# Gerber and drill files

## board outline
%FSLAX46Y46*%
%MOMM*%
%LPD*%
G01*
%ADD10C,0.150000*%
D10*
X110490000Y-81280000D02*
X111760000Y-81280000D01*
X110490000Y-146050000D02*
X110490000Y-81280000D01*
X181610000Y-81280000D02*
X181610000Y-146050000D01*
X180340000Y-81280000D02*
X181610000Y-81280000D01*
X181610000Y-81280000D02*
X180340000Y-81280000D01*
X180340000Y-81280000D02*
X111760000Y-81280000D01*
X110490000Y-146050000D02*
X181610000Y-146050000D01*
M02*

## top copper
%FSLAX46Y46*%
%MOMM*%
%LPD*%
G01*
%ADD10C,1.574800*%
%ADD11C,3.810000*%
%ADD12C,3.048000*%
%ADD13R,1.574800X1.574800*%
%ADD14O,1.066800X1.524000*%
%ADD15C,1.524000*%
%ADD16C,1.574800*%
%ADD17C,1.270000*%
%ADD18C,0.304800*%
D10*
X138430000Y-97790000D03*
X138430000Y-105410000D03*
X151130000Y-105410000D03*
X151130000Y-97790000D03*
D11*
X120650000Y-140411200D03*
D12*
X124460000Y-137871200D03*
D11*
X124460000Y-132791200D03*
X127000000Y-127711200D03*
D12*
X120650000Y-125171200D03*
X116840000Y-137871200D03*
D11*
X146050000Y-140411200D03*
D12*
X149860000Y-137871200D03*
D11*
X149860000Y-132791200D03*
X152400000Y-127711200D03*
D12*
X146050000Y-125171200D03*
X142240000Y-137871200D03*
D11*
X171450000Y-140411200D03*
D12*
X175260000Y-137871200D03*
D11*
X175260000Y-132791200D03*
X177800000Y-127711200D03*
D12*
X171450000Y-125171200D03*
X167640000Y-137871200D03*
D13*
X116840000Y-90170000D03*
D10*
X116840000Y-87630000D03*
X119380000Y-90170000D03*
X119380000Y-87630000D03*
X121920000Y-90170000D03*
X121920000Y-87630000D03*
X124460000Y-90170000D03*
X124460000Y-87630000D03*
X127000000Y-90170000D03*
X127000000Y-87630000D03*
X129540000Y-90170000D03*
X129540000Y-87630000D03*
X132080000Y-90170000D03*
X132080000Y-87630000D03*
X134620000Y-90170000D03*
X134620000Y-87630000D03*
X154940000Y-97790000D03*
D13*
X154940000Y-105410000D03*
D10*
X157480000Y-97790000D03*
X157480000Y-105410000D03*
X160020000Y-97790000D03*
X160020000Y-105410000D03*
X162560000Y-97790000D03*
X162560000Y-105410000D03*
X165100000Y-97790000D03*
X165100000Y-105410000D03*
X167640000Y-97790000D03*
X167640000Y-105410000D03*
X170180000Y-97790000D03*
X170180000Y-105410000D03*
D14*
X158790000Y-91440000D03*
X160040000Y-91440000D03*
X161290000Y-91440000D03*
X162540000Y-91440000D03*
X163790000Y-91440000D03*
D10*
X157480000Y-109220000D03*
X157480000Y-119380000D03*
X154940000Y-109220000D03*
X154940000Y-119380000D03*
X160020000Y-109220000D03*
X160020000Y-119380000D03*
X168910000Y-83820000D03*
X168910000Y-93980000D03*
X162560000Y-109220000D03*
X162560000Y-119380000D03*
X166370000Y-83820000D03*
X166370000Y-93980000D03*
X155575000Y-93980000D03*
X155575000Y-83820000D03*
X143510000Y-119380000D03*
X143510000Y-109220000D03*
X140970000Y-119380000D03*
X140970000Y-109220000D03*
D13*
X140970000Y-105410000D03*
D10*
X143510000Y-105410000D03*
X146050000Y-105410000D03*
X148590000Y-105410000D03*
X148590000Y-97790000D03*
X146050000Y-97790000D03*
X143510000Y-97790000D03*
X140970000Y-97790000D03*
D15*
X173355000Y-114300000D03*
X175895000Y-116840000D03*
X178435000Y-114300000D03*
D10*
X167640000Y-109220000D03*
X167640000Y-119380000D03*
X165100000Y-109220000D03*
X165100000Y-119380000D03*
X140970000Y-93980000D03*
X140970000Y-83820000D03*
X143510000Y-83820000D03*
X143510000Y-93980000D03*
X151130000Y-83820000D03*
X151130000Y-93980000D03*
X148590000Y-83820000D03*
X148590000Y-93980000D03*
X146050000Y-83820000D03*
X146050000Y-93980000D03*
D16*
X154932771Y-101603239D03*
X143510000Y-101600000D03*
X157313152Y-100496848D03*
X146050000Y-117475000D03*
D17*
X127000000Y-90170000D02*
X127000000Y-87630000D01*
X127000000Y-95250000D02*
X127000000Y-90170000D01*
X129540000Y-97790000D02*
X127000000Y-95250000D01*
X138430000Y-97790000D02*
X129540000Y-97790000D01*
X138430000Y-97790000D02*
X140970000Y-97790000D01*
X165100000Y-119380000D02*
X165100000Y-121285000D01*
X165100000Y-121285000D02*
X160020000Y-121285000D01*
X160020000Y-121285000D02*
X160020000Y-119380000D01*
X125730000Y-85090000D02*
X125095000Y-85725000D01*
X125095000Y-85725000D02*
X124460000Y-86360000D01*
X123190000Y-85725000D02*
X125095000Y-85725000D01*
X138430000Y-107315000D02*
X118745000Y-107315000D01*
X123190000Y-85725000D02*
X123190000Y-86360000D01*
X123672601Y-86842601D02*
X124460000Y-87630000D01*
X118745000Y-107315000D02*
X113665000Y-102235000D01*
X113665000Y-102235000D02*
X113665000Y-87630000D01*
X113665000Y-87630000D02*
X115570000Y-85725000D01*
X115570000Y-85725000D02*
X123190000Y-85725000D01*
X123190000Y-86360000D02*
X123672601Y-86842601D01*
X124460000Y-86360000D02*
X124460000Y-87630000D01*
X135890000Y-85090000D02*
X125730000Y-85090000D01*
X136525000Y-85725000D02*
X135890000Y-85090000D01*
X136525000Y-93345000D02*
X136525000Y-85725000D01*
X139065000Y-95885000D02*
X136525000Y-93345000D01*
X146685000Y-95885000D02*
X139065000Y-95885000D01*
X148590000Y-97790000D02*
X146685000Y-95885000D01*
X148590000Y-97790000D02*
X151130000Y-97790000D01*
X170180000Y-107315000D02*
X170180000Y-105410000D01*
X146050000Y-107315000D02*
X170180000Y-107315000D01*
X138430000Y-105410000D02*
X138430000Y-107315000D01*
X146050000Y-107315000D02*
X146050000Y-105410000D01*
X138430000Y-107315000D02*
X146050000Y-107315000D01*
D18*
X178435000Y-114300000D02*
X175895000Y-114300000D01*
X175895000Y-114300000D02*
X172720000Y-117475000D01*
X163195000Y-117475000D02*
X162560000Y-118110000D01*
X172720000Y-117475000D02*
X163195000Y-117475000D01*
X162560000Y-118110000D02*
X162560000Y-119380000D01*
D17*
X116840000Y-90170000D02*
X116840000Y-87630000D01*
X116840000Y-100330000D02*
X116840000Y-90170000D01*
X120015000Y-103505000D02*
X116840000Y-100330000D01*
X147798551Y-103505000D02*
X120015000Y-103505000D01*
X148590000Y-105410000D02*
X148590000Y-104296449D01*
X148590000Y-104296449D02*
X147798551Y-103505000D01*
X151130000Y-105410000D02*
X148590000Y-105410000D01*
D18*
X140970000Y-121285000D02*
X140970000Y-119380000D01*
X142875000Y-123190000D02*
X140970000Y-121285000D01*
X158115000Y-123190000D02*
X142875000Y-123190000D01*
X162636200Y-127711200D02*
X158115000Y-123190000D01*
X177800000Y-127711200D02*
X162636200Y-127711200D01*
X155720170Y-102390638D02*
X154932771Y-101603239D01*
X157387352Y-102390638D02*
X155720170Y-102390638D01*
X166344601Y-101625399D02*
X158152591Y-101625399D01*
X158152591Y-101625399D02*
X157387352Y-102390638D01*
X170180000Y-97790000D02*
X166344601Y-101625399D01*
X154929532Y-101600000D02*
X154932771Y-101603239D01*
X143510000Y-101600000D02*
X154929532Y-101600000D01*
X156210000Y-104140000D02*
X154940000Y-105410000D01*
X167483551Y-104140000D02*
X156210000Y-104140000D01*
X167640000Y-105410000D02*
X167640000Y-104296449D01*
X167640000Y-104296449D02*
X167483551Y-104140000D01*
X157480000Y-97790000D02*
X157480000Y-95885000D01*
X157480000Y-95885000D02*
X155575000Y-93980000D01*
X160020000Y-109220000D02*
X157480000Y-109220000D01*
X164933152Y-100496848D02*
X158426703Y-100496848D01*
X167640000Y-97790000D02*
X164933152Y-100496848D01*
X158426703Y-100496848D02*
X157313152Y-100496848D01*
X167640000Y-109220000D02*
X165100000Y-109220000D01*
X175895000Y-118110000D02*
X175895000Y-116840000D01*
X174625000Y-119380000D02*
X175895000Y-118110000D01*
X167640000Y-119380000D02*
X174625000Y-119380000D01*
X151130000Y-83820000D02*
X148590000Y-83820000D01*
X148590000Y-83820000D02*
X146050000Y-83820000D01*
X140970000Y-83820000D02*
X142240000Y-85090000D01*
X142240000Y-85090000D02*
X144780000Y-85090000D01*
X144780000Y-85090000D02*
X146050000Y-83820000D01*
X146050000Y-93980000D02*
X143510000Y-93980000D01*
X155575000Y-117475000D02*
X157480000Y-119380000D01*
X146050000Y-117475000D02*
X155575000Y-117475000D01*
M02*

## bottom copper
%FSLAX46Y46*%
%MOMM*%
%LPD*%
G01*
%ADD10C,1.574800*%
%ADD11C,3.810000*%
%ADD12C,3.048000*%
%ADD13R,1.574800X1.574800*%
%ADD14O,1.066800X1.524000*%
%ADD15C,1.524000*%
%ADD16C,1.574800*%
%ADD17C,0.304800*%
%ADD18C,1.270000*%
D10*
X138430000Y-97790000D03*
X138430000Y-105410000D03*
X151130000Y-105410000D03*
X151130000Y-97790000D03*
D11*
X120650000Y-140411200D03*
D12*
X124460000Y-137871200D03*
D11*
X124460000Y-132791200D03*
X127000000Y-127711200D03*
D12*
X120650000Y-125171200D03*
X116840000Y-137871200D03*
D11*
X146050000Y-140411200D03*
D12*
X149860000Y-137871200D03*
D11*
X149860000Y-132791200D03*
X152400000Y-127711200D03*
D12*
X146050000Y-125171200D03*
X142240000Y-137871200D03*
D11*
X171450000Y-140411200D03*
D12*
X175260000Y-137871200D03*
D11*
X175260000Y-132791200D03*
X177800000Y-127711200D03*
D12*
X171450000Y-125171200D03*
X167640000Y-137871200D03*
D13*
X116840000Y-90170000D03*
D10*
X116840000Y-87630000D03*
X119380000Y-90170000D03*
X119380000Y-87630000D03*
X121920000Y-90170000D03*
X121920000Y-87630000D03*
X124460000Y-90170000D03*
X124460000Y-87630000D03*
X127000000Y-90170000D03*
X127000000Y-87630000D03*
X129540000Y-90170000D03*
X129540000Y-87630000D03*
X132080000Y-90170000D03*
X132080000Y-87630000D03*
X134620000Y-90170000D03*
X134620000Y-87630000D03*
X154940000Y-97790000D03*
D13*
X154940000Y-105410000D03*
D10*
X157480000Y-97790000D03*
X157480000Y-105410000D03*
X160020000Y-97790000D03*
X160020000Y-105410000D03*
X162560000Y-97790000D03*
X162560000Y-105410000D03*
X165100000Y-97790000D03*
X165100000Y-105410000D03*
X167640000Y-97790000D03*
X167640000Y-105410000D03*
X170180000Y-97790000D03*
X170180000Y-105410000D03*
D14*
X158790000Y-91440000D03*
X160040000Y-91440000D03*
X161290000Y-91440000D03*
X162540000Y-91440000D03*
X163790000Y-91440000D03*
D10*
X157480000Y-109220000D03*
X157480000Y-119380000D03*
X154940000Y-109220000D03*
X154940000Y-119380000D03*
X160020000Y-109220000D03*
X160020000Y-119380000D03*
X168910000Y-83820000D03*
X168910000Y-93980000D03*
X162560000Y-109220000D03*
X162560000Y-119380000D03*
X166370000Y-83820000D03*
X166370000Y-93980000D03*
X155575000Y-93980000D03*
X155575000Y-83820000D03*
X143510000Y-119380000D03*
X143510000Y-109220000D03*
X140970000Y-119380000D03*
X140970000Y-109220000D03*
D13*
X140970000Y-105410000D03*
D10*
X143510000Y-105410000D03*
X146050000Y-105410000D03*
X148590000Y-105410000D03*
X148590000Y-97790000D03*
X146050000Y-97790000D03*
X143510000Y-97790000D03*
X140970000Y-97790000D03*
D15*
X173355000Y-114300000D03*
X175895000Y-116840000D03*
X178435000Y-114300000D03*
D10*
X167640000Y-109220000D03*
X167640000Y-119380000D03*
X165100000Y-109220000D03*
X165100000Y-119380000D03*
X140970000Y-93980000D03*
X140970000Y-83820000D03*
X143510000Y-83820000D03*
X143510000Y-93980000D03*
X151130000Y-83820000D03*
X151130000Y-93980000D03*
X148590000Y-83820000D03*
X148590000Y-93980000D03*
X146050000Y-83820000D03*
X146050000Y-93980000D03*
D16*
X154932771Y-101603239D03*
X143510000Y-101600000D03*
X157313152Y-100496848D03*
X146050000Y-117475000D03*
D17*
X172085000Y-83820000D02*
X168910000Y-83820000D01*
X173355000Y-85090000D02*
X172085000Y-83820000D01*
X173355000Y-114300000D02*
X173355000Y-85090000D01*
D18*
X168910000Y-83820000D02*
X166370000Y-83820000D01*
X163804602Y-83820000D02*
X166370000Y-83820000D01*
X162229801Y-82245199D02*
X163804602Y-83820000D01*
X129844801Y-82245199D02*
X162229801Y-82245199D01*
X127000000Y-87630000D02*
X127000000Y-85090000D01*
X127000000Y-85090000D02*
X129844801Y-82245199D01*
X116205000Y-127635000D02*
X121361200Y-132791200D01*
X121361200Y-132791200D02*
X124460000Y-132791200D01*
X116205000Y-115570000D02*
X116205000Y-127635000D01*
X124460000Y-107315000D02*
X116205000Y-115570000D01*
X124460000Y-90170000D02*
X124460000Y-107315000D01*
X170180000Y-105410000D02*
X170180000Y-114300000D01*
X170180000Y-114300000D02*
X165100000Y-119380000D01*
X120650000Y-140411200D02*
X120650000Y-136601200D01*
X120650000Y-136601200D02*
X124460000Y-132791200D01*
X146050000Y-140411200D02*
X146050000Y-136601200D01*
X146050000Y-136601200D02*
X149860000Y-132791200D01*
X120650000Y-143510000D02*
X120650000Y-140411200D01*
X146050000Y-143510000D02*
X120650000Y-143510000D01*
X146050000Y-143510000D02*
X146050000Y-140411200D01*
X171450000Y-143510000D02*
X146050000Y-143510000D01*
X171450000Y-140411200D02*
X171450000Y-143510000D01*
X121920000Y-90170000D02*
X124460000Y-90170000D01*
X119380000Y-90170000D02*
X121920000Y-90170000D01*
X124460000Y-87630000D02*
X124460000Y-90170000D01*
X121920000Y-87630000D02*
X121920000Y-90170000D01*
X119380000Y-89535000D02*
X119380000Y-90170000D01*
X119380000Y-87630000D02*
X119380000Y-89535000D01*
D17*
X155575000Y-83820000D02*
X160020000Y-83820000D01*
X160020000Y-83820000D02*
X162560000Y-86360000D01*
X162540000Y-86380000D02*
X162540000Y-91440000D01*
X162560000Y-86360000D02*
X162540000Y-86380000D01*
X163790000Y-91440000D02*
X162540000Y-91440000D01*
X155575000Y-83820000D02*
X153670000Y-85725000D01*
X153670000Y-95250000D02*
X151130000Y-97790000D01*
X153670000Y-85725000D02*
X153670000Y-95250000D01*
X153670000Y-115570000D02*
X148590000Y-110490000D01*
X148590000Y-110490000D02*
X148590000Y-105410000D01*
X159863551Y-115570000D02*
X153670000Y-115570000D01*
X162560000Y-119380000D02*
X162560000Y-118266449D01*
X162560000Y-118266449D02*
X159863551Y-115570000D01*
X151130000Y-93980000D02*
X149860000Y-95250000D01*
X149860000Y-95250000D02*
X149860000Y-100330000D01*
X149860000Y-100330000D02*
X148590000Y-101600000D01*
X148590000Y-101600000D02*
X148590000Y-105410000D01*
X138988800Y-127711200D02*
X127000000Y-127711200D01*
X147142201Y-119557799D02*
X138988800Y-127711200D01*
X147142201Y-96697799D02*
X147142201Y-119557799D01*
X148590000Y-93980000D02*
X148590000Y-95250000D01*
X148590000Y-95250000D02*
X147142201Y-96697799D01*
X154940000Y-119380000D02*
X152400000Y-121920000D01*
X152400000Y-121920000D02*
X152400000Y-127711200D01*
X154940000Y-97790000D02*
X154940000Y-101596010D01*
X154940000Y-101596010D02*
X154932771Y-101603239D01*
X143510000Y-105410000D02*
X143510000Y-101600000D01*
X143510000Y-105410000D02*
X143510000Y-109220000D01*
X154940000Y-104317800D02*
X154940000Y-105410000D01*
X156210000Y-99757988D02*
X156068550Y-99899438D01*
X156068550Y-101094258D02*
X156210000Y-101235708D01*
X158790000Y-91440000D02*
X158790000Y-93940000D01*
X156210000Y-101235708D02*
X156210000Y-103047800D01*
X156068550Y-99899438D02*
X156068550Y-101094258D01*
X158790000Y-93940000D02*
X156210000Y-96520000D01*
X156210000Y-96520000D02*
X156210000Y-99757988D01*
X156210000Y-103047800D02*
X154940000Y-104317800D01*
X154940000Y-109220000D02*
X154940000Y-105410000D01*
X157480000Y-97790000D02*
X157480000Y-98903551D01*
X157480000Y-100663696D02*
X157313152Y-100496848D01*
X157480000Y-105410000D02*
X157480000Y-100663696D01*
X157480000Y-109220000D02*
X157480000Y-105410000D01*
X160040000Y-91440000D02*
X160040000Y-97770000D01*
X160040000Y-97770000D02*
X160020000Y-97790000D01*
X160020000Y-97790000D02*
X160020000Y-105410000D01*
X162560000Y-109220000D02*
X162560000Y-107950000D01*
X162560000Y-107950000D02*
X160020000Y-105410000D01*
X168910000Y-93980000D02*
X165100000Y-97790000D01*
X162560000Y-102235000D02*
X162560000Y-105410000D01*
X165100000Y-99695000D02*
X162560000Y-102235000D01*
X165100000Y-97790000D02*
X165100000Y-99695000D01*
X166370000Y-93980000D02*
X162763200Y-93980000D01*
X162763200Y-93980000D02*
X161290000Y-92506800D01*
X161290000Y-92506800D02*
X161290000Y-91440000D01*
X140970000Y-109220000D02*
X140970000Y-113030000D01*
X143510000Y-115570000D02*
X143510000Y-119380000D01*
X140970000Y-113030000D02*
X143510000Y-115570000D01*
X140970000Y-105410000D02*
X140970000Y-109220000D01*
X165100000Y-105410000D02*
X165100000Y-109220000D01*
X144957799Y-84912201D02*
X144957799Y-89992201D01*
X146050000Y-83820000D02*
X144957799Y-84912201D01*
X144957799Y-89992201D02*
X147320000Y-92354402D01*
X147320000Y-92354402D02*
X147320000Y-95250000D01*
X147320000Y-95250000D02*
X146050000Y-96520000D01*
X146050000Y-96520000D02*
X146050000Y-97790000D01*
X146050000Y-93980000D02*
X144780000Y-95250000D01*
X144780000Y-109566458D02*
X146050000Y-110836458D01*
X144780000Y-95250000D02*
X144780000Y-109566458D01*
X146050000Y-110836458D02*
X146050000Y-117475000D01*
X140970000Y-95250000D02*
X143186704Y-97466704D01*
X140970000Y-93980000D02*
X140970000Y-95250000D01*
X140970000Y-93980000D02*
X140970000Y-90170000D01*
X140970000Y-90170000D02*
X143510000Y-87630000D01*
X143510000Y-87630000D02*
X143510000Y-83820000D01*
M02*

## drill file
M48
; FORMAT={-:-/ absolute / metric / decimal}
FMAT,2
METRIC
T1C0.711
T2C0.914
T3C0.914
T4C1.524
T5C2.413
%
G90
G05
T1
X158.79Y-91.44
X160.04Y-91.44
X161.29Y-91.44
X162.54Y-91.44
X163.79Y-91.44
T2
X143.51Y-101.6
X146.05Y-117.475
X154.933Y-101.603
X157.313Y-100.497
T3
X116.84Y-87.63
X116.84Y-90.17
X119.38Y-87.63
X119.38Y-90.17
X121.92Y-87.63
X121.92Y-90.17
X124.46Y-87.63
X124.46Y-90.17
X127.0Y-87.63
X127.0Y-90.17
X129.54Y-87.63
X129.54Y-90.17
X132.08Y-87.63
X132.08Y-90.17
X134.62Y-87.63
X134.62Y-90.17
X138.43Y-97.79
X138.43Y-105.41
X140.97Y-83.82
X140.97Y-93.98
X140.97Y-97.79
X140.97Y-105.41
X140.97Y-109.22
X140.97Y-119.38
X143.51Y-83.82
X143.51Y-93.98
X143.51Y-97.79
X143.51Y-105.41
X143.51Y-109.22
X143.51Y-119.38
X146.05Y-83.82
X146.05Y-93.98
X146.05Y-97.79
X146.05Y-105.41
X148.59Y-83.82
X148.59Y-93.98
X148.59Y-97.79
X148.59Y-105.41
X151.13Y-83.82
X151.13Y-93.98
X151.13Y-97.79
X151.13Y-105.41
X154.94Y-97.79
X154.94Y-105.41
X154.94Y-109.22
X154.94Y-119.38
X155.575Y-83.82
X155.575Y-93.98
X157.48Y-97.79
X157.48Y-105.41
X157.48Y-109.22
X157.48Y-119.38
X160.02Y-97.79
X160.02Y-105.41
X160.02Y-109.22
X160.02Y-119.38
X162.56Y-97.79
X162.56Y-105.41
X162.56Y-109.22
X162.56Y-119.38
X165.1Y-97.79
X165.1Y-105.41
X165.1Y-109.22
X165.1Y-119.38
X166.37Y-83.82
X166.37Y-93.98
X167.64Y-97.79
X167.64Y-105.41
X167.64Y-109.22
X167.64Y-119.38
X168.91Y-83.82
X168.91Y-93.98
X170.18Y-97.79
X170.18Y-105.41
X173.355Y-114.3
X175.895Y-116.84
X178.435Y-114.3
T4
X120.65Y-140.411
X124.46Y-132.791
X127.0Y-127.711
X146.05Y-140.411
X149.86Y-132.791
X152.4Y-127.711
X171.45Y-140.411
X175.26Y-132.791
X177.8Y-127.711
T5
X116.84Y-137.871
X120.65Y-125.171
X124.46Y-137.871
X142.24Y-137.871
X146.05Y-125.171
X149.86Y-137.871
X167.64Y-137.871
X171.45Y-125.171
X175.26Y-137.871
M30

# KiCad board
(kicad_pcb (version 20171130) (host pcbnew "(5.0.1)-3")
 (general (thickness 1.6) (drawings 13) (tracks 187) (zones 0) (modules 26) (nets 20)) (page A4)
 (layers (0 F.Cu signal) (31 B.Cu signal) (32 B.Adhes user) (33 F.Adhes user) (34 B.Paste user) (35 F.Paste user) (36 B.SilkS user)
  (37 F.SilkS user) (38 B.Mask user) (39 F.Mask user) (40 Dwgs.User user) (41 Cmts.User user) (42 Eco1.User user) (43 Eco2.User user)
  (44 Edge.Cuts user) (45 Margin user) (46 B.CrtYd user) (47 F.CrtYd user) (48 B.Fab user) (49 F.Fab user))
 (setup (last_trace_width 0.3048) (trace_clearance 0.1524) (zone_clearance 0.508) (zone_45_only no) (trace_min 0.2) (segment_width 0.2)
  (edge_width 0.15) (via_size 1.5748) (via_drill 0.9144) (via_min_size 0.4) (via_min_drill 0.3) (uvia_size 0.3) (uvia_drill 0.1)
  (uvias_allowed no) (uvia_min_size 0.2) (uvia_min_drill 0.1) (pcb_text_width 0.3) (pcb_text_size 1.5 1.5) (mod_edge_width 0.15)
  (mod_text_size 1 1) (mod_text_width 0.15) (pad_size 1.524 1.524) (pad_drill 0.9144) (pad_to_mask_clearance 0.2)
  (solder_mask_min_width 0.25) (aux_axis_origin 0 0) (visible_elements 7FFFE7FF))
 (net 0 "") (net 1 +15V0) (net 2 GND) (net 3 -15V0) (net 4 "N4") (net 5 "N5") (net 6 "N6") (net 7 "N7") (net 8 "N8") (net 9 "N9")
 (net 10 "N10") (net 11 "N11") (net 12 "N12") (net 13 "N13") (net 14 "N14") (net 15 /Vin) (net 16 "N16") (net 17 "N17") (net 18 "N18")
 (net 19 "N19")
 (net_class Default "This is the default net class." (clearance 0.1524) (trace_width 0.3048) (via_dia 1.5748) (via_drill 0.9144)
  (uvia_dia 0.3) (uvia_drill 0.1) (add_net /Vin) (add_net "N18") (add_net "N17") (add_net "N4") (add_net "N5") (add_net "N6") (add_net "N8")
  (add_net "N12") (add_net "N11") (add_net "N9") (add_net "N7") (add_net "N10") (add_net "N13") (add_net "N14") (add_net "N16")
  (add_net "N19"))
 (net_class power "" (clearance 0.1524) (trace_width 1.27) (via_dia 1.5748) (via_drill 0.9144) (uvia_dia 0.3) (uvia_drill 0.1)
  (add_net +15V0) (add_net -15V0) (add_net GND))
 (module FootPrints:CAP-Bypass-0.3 (layer F.Cu) (at 138.43 101.6 270)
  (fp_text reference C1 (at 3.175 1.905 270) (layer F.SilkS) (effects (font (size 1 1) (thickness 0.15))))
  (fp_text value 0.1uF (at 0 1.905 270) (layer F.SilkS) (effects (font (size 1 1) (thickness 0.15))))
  (pad 1 thru_hole circle (at -3.81 0 270) (size 1.5748 1.5748) (drill 0.9144) (layers *.Cu *.Mask F.SilkS) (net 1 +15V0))
  (pad 2 thru_hole circle (at 3.81 0 270) (size 1.5748 1.5748) (drill 0.9144) (layers *.Cu *.Mask F.SilkS) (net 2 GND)))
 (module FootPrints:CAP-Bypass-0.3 (layer F.Cu) (at 151.13 101.6 90)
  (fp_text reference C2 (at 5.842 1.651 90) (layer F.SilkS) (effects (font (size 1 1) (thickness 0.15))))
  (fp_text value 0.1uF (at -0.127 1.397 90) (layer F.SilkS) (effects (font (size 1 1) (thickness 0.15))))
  (pad 1 thru_hole circle (at -3.81 0 90) (size 1.5748 1.5748) (drill 0.9144) (layers *.Cu *.Mask F.SilkS) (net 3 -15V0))
  (pad 2 thru_hole circle (at 3.81 0 90) (size 1.5748 1.5748) (drill 0.9144) (layers *.Cu *.Mask F.SilkS) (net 2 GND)))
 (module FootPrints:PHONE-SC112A (layer F.Cu) (at 120.65 146.05 270)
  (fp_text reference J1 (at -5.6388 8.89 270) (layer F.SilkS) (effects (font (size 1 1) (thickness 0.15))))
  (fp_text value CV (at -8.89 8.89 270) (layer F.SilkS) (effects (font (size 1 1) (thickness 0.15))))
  (pad 1 thru_hole circle (at -5.6388 0 270) (size 3.81 3.81) (drill 1.524) (layers *.Cu *.Mask F.SilkS) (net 2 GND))
  (pad "" thru_hole circle (at -8.1788 -3.81 270) (size 3.048 3.048) (drill 2.413) (layers *.Cu *.Mask F.SilkS))
  (pad 2 thru_hole circle (at -13.2588 -3.81 270) (size 3.81 3.81) (drill 1.524) (layers *.Cu *.Mask F.SilkS) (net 2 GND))
  (pad 3 thru_hole circle (at -18.3388 -6.35 270) (size 3.81 3.81) (drill 1.524) (layers *.Cu *.Mask F.SilkS) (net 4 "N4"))
  (pad "" thru_hole circle (at -20.8788 0 270) (size 3.048 3.048) (drill 2.413) (layers *.Cu *.Mask F.SilkS))
  (pad "" thru_hole circle (at -8.1788 3.81 270) (size 3.048 3.048) (drill 2.413) (layers *.Cu *.Mask F.SilkS)))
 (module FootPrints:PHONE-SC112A (layer F.Cu) (at 146.05 146.05 270)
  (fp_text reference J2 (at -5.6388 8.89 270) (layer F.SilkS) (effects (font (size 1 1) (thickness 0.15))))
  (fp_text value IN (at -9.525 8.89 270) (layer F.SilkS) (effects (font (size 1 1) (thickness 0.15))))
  (pad 1 thru_hole circle (at -5.6388 0 270) (size 3.81 3.81) (drill 1.524) (layers *.Cu *.Mask F.SilkS) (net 2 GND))
  (pad "" thru_hole circle (at -8.1788 -3.81 270) (size 3.048 3.048) (drill 2.413) (layers *.Cu *.Mask F.SilkS))
  (pad 2 thru_hole circle (at -13.2588 -3.81 270) (size 3.81 3.81) (drill 1.524) (layers *.Cu *.Mask F.SilkS) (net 2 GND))
  (pad 3 thru_hole circle (at -18.3388 -6.35 270) (size 3.81 3.81) (drill 1.524) (layers *.Cu *.Mask F.SilkS) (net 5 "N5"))
  (pad "" thru_hole circle (at -20.8788 0 270) (size 3.048 3.048) (drill 2.413) (layers *.Cu *.Mask F.SilkS))
  (pad "" thru_hole circle (at -8.1788 3.81 270) (size 3.048 3.048) (drill 2.413) (layers *.Cu *.Mask F.SilkS)))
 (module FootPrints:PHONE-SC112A (layer F.Cu) (at 171.45 146.05 270)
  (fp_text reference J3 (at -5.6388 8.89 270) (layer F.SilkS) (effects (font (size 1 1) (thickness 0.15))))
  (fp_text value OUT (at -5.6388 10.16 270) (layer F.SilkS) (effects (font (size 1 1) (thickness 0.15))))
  (pad 1 thru_hole circle (at -5.6388 0 270) (size 3.81 3.81) (drill 1.524) (layers *.Cu *.Mask F.SilkS) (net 2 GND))
  (pad "" thru_hole circle (at -8.1788 -3.81 270) (size 3.048 3.048) (drill 2.413) (layers *.Cu *.Mask F.SilkS))
  (pad 2 thru_hole circle (at -13.2588 -3.81 270) (size 3.81 3.81) (drill 1.524) (layers *.Cu *.Mask F.SilkS))
  (pad 3 thru_hole circle (at -18.3388 -6.35 270) (size 3.81 3.81) (drill 1.524) (layers *.Cu *.Mask F.SilkS) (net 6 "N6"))
  (pad "" thru_hole circle (at -20.8788 0 270) (size 3.048 3.048) (drill 2.413) (layers *.Cu *.Mask F.SilkS))
  (pad "" thru_hole circle (at -8.1788 3.81 270) (size 3.048 3.048) (drill 2.413) (layers *.Cu *.Mask F.SilkS)))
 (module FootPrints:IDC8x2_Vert (layer F.Cu) (at 125.73 88.9 180)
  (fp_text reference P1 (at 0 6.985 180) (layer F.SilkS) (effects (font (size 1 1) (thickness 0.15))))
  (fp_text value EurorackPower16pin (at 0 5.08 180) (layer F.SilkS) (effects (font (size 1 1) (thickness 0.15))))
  (pad 1 thru_hole rect (at 8.89 -1.27 180) (size 1.5748 1.5748) (drill 0.9144) (layers *.Cu *.Mask F.SilkS) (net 3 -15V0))
  (pad 2 thru_hole circle (at 8.89 1.27 180) (size 1.5748 1.5748) (drill 0.9144) (layers *.Cu *.Mask F.SilkS) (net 3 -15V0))
  (pad 3 thru_hole circle (at 6.35 -1.27 180) (size 1.5748 1.5748) (drill 0.9144) (layers *.Cu *.Mask F.SilkS) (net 2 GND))
  (pad 4 thru_hole circle (at 6.35 1.27 180) (size 1.5748 1.5748) (drill 0.9144) (layers *.Cu *.Mask F.SilkS) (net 2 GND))
  (pad 5 thru_hole circle (at 3.81 -1.27 180) (size 1.5748 1.5748) (drill 0.9144) (layers *.Cu *.Mask F.SilkS) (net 2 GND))
  (pad 6 thru_hole circle (at 3.81 1.27 180) (size 1.5748 1.5748) (drill 0.9144) (layers *.Cu *.Mask F.SilkS) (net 2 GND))
  (pad 7 thru_hole circle (at 1.27 -1.27 180) (size 1.5748 1.5748) (drill 0.9144) (layers *.Cu *.Mask F.SilkS) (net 2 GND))
  (pad 8 thru_hole circle (at 1.27 1.27 180) (size 1.5748 1.5748) (drill 0.9144) (layers *.Cu *.Mask F.SilkS) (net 2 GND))
  (pad 9 thru_hole circle (at -1.27 -1.27 180) (size 1.5748 1.5748) (drill 0.9144) (layers *.Cu *.Mask F.SilkS) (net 1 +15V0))
  (pad 10 thru_hole circle (at -1.27 1.27 180) (size 1.5748 1.5748) (drill 0.9144) (layers *.Cu *.Mask F.SilkS) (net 1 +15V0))
  (pad 11 thru_hole circle (at -3.81 -1.27 180) (size 1.5748 1.5748) (drill 0.9144) (layers *.Cu *.Mask F.SilkS))
  (pad 12 thru_hole circle (at -3.81 1.27 180) (size 1.5748 1.5748) (drill 0.9144) (layers *.Cu *.Mask F.SilkS))
  (pad 13 thru_hole circle (at -6.35 -1.27 180) (size 1.5748 1.5748) (drill 0.9144) (layers *.Cu *.Mask F.SilkS))
  (pad 14 thru_hole circle (at -6.35 1.27 180) (size 1.5748 1.5748) (drill 0.9144) (layers *.Cu *.Mask F.SilkS))
  (pad 15 thru_hole circle (at -8.89 -1.27 180) (size 1.5748 1.5748) (drill 0.9144) (layers *.Cu *.Mask F.SilkS))
  (pad 16 thru_hole circle (at -8.89 1.27 180) (size 1.5748 1.5748) (drill 0.9144) (layers *.Cu *.Mask F.SilkS)))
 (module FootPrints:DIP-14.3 (layer F.Cu) (at 162.56 101.6)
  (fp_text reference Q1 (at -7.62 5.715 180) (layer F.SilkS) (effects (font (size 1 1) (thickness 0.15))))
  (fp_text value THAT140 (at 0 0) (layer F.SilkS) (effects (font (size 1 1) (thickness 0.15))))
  (pad 14 thru_hole circle (at -7.62 -3.81) (size 1.5748 1.5748) (drill 0.9144) (layers *.Cu *.Mask F.SilkS) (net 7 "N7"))
  (pad 1 thru_hole rect (at -7.62 3.81) (size 1.5748 1.5748) (drill 0.9144) (layers *.Cu *.Mask F.SilkS) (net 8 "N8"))
  (pad 13 thru_hole circle (at -5.08 -3.81) (size 1.5748 1.5748) (drill 0.9144) (layers *.Cu *.Mask F.SilkS) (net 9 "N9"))
  (pad 2 thru_hole circle (at -5.08 3.81) (size 1.5748 1.5748) (drill 0.9144) (layers *.Cu *.Mask F.SilkS) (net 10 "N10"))
  (pad 12 thru_hole circle (at -2.54 -3.81) (size 1.5748 1.5748) (drill 0.9144) (layers *.Cu *.Mask F.SilkS) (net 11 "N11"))
  (pad 3 thru_hole circle (at -2.54 3.81) (size 1.5748 1.5748) (drill 0.9144) (layers *.Cu *.Mask F.SilkS) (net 11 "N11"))
  (pad 11 thru_hole circle (at 0 -3.81) (size 1.5748 1.5748) (drill 0.9144) (layers *.Cu *.Mask F.SilkS))
  (pad 4 thru_hole circle (at 0 3.81) (size 1.5748 1.5748) (drill 0.9144) (layers *.Cu *.Mask F.SilkS) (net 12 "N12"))
  (pad 10 thru_hole circle (at 2.54 -3.81) (size 1.5748 1.5748) (drill 0.9144) (layers *.Cu *.Mask F.SilkS) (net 12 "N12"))
  (pad 5 thru_hole circle (at 2.54 3.81) (size 1.5748 1.5748) (drill 0.9144) (layers *.Cu *.Mask F.SilkS) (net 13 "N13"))
  (pad 9 thru_hole circle (at 5.08 -3.81) (size 1.5748 1.5748) (drill 0.9144) (layers *.Cu *.Mask F.SilkS) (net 10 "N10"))
  (pad 6 thru_hole circle (at 5.08 3.81) (size 1.5748 1.5748) (drill 0.9144) (layers *.Cu *.Mask F.SilkS) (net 8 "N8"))
  (pad 8 thru_hole circle (at 7.62 -3.81) (size 1.5748 1.5748) (drill 0.9144) (layers *.Cu *.Mask F.SilkS) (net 7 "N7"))
  (pad 7 thru_hole circle (at 7.62 3.81) (size 1.5748 1.5748) (drill 0.9144) (layers *.Cu *.Mask F.SilkS) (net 2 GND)))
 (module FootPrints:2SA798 (layer F.Cu) (at 161.29 91.44)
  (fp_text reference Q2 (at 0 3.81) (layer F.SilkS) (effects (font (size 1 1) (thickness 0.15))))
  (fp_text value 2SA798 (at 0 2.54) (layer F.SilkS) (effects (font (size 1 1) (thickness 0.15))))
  (pad 1 thru_hole oval (at -2.5 0) (size 1.0668 1.524) (drill 0.7112) (layers *.Cu *.Mask F.SilkS) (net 8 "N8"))
  (pad 2 thru_hole oval (at -1.25 0) (size 1.0668 1.524) (drill 0.7112) (layers *.Cu *.Mask F.SilkS) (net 11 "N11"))
  (pad 3 thru_hole oval (at 0 0) (size 1.0668 1.524) (drill 0.7112) (layers *.Cu *.Mask F.SilkS) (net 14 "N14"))
  (pad 4 thru_hole oval (at 1.25 0) (size 1.0668 1.524) (drill 0.7112) (layers *.Cu *.Mask F.SilkS) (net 2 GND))
  (pad 5 thru_hole oval (at 2.5 0) (size 1.0668 1.524) (drill 0.7112) (layers *.Cu *.Mask F.SilkS) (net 2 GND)))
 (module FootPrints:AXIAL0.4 (layer F.Cu) (at 157.48 114.3 270)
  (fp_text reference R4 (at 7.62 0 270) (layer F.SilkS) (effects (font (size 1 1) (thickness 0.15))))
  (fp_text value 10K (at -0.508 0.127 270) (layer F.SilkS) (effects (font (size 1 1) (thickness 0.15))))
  (pad 1 thru_hole circle (at -5.08 0 270) (size 1.5748 1.5748) (drill 0.9144) (layers *.Cu *.Mask F.SilkS) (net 10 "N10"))
  (pad 2 thru_hole circle (at 5.08 0 270) (size 1.5748 1.5748) (drill 0.9144) (layers *.Cu *.Mask F.SilkS) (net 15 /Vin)))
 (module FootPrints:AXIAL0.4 (layer F.Cu) (at 154.94 114.3 270)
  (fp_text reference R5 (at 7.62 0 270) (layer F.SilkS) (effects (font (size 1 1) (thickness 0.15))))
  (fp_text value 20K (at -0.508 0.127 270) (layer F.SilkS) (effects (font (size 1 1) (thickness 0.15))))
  (pad 1 thru_hole circle (at -5.08 0 270) (size 1.5748 1.5748) (drill 0.9144) (layers *.Cu *.Mask F.SilkS) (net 8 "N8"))
  (pad 2 thru_hole circle (at 5.08 0 270) (size 1.5748 1.5748) (drill 0.9144) (layers *.Cu *.Mask F.SilkS) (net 5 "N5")))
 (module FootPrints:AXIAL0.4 (layer F.Cu) (at 160.02 114.3 270)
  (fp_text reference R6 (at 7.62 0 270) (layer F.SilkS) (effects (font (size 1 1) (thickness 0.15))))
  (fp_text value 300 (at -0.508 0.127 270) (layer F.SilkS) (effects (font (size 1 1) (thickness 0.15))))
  (pad 1 thru_hole circle (at -5.08 0 270) (size 1.5748 1.5748) (drill 0.9144) (layers *.Cu *.Mask F.SilkS) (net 10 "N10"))
  (pad 2 thru_hole circle (at 5.08 0 270) (size 1.5748 1.5748) (drill 0.9144) (layers *.Cu *.Mask F.SilkS) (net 2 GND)))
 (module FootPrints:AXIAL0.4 (layer F.Cu) (at 168.91 88.9 270)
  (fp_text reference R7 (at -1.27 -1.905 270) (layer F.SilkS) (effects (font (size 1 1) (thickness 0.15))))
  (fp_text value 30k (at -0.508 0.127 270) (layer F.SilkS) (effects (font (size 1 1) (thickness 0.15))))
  (pad 1 thru_hole circle (at -5.08 0 270) (size 1.5748 1.5748) (drill 0.9144) (layers *.Cu *.Mask F.SilkS) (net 1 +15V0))
  (pad 2 thru_hole circle (at 5.08 0 270) (size 1.5748 1.5748) (drill 0.9144) (layers *.Cu *.Mask F.SilkS) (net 12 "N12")))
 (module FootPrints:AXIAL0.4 (layer F.Cu) (at 162.56 114.3 270)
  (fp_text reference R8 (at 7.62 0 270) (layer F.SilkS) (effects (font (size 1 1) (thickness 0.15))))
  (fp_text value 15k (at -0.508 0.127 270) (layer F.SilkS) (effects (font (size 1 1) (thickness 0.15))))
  (pad 1 thru_hole circle (at -5.08 0 270) (size 1.5748 1.5748) (drill 0.9144) (layers *.Cu *.Mask F.SilkS) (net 11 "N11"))
  (pad 2 thru_hole circle (at 5.08 0 270) (size 1.5748 1.5748) (drill 0.9144) (layers *.Cu *.Mask F.SilkS) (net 3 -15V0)))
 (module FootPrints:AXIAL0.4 (layer F.Cu) (at 166.37 88.9 270)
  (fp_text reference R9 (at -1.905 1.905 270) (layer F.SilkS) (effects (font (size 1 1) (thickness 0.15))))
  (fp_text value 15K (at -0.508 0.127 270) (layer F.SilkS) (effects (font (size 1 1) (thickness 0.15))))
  (pad 1 thru_hole circle (at -5.08 0 270) (size 1.5748 1.5748) (drill 0.9144) (layers *.Cu *.Mask F.SilkS) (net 1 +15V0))
  (pad 2 thru_hole circle (at 5.08 0 270) (size 1.5748 1.5748) (drill 0.9144) (layers *.Cu *.Mask F.SilkS) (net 14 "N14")))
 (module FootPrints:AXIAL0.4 (layer F.Cu) (at 155.575 88.9 90)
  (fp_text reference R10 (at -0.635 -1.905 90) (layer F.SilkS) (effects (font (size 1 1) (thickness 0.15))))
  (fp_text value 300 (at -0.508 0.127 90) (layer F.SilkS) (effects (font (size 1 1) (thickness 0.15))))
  (pad 1 thru_hole circle (at -5.08 0 90) (size 1.5748 1.5748) (drill 0.9144) (layers *.Cu *.Mask F.SilkS) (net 9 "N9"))
  (pad 2 thru_hole circle (at 5.08 0 90) (size 1.5748 1.5748) (drill 0.9144) (layers *.Cu *.Mask F.SilkS) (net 2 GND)))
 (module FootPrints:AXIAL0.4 (layer F.Cu) (at 143.51 114.3 90)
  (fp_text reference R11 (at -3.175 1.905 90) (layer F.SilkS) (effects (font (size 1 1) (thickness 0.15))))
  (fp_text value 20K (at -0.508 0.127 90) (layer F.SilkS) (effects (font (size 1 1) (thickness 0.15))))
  (pad 1 thru_hole circle (at -5.08 0 90) (size 1.5748 1.5748) (drill 0.9144) (layers *.Cu *.Mask F.SilkS) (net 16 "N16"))
  (pad 2 thru_hole circle (at 5.08 0 90) (size 1.5748 1.5748) (drill 0.9144) (layers *.Cu *.Mask F.SilkS) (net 7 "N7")))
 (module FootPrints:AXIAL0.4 (layer F.Cu) (at 140.97 114.3 90)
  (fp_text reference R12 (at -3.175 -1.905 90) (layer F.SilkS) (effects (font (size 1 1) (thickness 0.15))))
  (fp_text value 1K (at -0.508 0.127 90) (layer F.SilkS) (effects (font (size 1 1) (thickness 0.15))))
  (pad 1 thru_hole circle (at -5.08 0 90) (size 1.5748 1.5748) (drill 0.9144) (layers *.Cu *.Mask F.SilkS) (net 6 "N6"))
  (pad 2 thru_hole circle (at 5.08 0 90) (size 1.5748 1.5748) (drill 0.9144) (layers *.Cu *.Mask F.SilkS) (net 16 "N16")))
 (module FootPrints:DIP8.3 (layer F.Cu) (at 144.78 101.6)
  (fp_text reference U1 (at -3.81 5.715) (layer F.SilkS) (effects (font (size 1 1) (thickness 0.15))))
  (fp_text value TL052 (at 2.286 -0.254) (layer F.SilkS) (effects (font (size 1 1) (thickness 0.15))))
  (pad 1 thru_hole rect (at -3.81 3.81) (size 1.5748 1.5748) (drill 0.9144) (layers *.Cu *.Mask F.SilkS) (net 16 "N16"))
  (pad 2 thru_hole circle (at -1.27 3.81) (size 1.5748 1.5748) (drill 0.9144) (layers *.Cu *.Mask F.SilkS) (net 7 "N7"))
  (pad 3 thru_hole circle (at 1.27 3.81) (size 1.5748 1.5748) (drill 0.9144) (layers *.Cu *.Mask F.SilkS) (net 2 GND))
  (pad 4 thru_hole circle (at 3.81 3.81) (size 1.5748 1.5748) (drill 0.9144) (layers *.Cu *.Mask F.SilkS) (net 3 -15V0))
  (pad 5 thru_hole circle (at 3.81 -3.81) (size 1.5748 1.5748) (drill 0.9144) (layers *.Cu *.Mask F.SilkS) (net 2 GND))
  (pad 6 thru_hole circle (at 1.27 -3.81) (size 1.5748 1.5748) (drill 0.9144) (layers *.Cu *.Mask F.SilkS) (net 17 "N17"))
  (pad 7 thru_hole circle (at -1.27 -3.81) (size 1.5748 1.5748) (drill 0.9144) (layers *.Cu *.Mask F.SilkS) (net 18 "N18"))
  (pad 8 thru_hole circle (at -3.81 -3.81) (size 1.5748 1.5748) (drill 0.9144) (layers *.Cu *.Mask F.SilkS) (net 1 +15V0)))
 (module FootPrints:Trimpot (layer F.Cu) (at 175.895 119.38)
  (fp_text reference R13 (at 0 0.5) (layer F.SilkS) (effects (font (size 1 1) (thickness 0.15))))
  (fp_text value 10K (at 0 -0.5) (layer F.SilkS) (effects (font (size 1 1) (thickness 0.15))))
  (pad 1 thru_hole circle (at -2.54 -5.08) (size 1.524 1.524) (drill 0.9144) (layers *.Cu *.Mask) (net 1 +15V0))
  (pad 2 thru_hole circle (at 0 -2.54) (size 1.524 1.524) (drill 0.9144) (layers *.Cu *.Mask) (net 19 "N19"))
  (pad 3 thru_hole circle (at 2.54 -5.08) (size 1.524 1.524) (drill 0.9144) (layers *.Cu *.Mask) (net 3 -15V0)))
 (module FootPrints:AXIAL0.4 (layer F.Cu) (at 167.64 114.3 270)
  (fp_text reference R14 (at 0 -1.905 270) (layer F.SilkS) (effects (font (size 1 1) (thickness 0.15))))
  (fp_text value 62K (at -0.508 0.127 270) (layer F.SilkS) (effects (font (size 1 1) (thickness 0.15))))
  (pad 1 thru_hole circle (at -5.08 0 270) (size 1.5748 1.5748) (drill 0.9144) (layers *.Cu *.Mask F.SilkS) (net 13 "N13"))
  (pad 2 thru_hole circle (at 5.08 0 270) (size 1.5748 1.5748) (drill 0.9144) (layers *.Cu *.Mask F.SilkS) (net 19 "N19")))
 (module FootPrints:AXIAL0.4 (layer F.Cu) (at 165.1 114.3 270)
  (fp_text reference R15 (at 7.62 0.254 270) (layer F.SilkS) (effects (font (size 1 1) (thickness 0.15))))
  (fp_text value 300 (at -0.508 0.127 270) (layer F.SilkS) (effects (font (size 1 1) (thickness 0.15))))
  (pad 1 thru_hole circle (at -5.08 0 270) (size 1.5748 1.5748) (drill 0.9144) (layers *.Cu *.Mask F.SilkS) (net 13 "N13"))
  (pad 2 thru_hole circle (at 5.08 0 270) (size 1.5748 1.5748) (drill 0.9144) (layers *.Cu *.Mask F.SilkS) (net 2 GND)))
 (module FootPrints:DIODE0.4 (layer F.Cu) (at 140.97 88.9 90)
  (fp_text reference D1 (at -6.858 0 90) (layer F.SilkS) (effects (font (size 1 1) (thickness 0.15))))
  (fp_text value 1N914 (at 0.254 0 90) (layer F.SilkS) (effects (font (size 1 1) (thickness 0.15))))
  (pad 1 thru_hole circle (at -5.08 0 90) (size 1.5748 1.5748) (drill 0.9144) (layers *.Cu *.Mask F.SilkS) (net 18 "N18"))
  (pad 2 thru_hole circle (at 5.08 0 90) (size 1.5748 1.5748) (drill 0.9144) (layers *.Cu *.Mask F.SilkS) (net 17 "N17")))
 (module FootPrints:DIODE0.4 (layer F.Cu) (at 143.51 88.9 90)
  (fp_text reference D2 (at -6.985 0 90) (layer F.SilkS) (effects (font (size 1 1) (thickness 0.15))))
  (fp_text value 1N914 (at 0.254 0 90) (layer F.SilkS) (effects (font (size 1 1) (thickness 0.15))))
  (pad 2 thru_hole circle (at 5.08 0 90) (size 1.5748 1.5748) (drill 0.9144) (layers *.Cu *.Mask F.SilkS) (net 18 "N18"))
  (pad 1 thru_hole circle (at -5.08 0 90) (size 1.5748 1.5748) (drill 0.9144) (layers *.Cu *.Mask F.SilkS) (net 15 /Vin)))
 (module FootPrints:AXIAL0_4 (layer F.Cu) (at 151.13 88.9 270)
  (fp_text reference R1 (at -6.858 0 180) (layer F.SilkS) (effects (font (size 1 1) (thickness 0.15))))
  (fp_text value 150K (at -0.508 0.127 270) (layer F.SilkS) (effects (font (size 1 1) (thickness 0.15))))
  (pad 1 thru_hole circle (at -5.08 0 270) (size 1.5748 1.5748) (drill 0.9144) (layers *.Cu *.Mask F.SilkS) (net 17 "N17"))
  (pad 2 thru_hole circle (at 5.08 0 270) (size 1.5748 1.5748) (drill 0.9144) (layers *.Cu *.Mask F.SilkS) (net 3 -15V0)))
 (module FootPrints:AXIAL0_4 (layer F.Cu) (at 148.59 88.9 270)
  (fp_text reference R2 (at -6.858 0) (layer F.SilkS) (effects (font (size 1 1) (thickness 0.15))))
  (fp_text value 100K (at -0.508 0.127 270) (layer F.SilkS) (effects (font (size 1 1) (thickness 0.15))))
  (pad 1 thru_hole circle (at -5.08 0 270) (size 1.5748 1.5748) (drill 0.9144) (layers *.Cu *.Mask F.SilkS) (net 17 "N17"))
  (pad 2 thru_hole circle (at 5.08 0 270) (size 1.5748 1.5748) (drill 0.9144) (layers *.Cu *.Mask F.SilkS) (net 4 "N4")))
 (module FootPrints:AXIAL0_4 (layer F.Cu) (at 146.05 88.9 90)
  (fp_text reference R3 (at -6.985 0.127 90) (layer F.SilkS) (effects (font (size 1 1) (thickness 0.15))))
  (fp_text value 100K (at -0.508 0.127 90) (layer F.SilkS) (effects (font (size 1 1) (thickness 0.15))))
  (pad 2 thru_hole circle (at 5.08 0 90) (size 1.5748 1.5748) (drill 0.9144) (layers *.Cu *.Mask F.SilkS) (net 17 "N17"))
  (pad 1 thru_hole circle (at -5.08 0 90) (size 1.5748 1.5748) (drill 0.9144) (layers *.Cu *.Mask F.SilkS) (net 15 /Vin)))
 (gr_line (start 110.49 81.28) (end 111.76 81.28) (angle 90) (layer Edge.Cuts) (width 0.15))
 (gr_line (start 110.49 146.05) (end 110.49 81.28) (angle 90) (layer Edge.Cuts) (width 0.15))
 (gr_line (start 181.61 81.28) (end 181.61 146.05) (angle 90) (layer Edge.Cuts) (width 0.15))
 (gr_line (start 180.34 81.28) (end 181.61 81.28) (angle 90) (layer Edge.Cuts) (width 0.15))
 (gr_line (start 181.61 81.28) (end 180.34 81.28) (angle 90) (layer Edge.Cuts) (width 0.15))
 (gr_line (start 180.34 81.28) (end 111.76 81.28) (angle 90) (layer Edge.Cuts) (width 0.15))
 (gr_line (start 110.49 146.05) (end 181.61 146.05) (angle 90) (layer Edge.Cuts) (width 0.15))
 (segment (start 172.085 83.82) (end 168.91 83.82) (width 0.3048) (layer B.Cu) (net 1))
 (segment (start 173.355 85.09) (end 172.085 83.82) (width 0.3048) (layer B.Cu) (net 1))
 (segment (start 173.355 114.3) (end 173.355 85.09) (width 0.3048) (layer B.Cu) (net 1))
 (segment (start 168.91 83.82) (end 166.37 83.82) (width 1.27) (layer B.Cu) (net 1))
 (segment (start 127 90.17) (end 127 87.63) (width 1.27) (layer F.Cu) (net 1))
 (segment (start 127 95.25) (end 127 90.17) (width 1.27) (layer F.Cu) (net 1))
 (segment (start 129.54 97.79) (end 127 95.25) (width 1.27) (layer F.Cu) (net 1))
 (segment (start 138.43 97.79) (end 129.54 97.79) (width 1.27) (layer F.Cu) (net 1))
 (segment (start 138.43 97.79) (end 140.97 97.79) (width 1.27) (layer F.Cu) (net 1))
 (segment (start 163.804602 83.82) (end 166.37 83.82) (width 1.27) (layer B.Cu) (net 1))
 (segment (start 162.229801 82.245199) (end 163.804602 83.82) (width 1.27) (layer B.Cu) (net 1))
 (segment (start 129.844801 82.245199) (end 162.229801 82.245199) (width 1.27) (layer B.Cu) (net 1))
 (segment (start 127 87.63) (end 127 85.09) (width 1.27) (layer B.Cu) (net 1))
 (segment (start 127 85.09) (end 129.844801 82.245199) (width 1.27) (layer B.Cu) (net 1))
 (segment (start 116.205 127.635) (end 121.3612 132.7912) (width 1.27) (layer B.Cu) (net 2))
 (segment (start 121.3612 132.7912) (end 124.46 132.7912) (width 1.27) (layer B.Cu) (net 2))
 (segment (start 116.205 115.57) (end 116.205 127.635) (width 1.27) (layer B.Cu) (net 2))
 (segment (start 124.46 107.315) (end 116.205 115.57) (width 1.27) (layer B.Cu) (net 2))
 (segment (start 124.46 90.17) (end 124.46 107.315) (width 1.27) (layer B.Cu) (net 2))
 (segment (start 170.18 105.41) (end 170.18 114.3) (width 1.27) (layer B.Cu) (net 2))
 (segment (start 170.18 114.3) (end 165.1 119.38) (width 1.27) (layer B.Cu) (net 2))
 (segment (start 120.65 140.4112) (end 120.65 136.6012) (width 1.27) (layer B.Cu) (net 2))
 (segment (start 120.65 136.6012) (end 124.46 132.7912) (width 1.27) (layer B.Cu) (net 2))
 (segment (start 146.05 140.4112) (end 146.05 136.6012) (width 1.27) (layer B.Cu) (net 2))
 (segment (start 146.05 136.6012) (end 149.86 132.7912) (width 1.27) (layer B.Cu) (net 2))
 (segment (start 120.65 143.51) (end 120.65 140.4112) (width 1.27) (layer B.Cu) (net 2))
 (segment (start 146.05 143.51) (end 120.65 143.51) (width 1.27) (layer B.Cu) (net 2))
 (segment (start 146.05 143.51) (end 146.05 140.4112) (width 1.27) (layer B.Cu) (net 2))
 (segment (start 171.45 143.51) (end 146.05 143.51) (width 1.27) (layer B.Cu) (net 2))
 (segment (start 171.45 140.4112) (end 171.45 143.51) (width 1.27) (layer B.Cu) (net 2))
 (segment (start 165.1 119.38) (end 165.1 121.285) (width 1.27) (layer F.Cu) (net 2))
 (segment (start 165.1 121.285) (end 160.02 121.285) (width 1.27) (layer F.Cu) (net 2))
 (segment (start 160.02 121.285) (end 160.02 119.38) (width 1.27) (layer F.Cu) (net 2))
 (segment (start 125.73 85.09) (end 125.095 85.725) (width 1.27) (layer F.Cu) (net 2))
 (segment (start 125.095 85.725) (end 124.46 86.36) (width 1.27) (layer F.Cu) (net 2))
 (segment (start 123.19 85.725) (end 125.095 85.725) (width 1.27) (layer F.Cu) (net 2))
 (segment (start 138.43 107.315) (end 118.745 107.315) (width 1.27) (layer F.Cu) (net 2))
 (segment (start 123.19 85.725) (end 123.19 86.36) (width 1.27) (layer F.Cu) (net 2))
 (segment (start 123.672601 86.842601) (end 124.46 87.63) (width 1.27) (layer F.Cu) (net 2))
 (segment (start 118.745 107.315) (end 113.665 102.235) (width 1.27) (layer F.Cu) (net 2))
 (segment (start 113.665 102.235) (end 113.665 87.63) (width 1.27) (layer F.Cu) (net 2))
 (segment (start 113.665 87.63) (end 115.57 85.725) (width 1.27) (layer F.Cu) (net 2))
 (segment (start 115.57 85.725) (end 123.19 85.725) (width 1.27) (layer F.Cu) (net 2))
 (segment (start 123.19 86.36) (end 123.672601 86.842601) (width 1.27) (layer F.Cu) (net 2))
 (segment (start 124.46 86.36) (end 124.46 87.63) (width 1.27) (layer F.Cu) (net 2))
 (segment (start 135.89 85.09) (end 125.73 85.09) (width 1.27) (layer F.Cu) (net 2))
 (segment (start 136.525 85.725) (end 135.89 85.09) (width 1.27) (layer F.Cu) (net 2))
 (segment (start 136.525 93.345) (end 136.525 85.725) (width 1.27) (layer F.Cu) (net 2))
 (segment (start 139.065 95.885) (end 136.525 93.345) (width 1.27) (layer F.Cu) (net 2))
 (segment (start 146.685 95.885) (end 139.065 95.885) (width 1.27) (layer F.Cu) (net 2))
 (segment (start 148.59 97.79) (end 146.685 95.885) (width 1.27) (layer F.Cu) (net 2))
 (segment (start 148.59 97.79) (end 151.13 97.79) (width 1.27) (layer F.Cu) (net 2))
 (segment (start 170.18 107.315) (end 170.18 105.41) (width 1.27) (layer F.Cu) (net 2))
 (segment (start 146.05 107.315) (end 170.18 107.315) (width 1.27) (layer F.Cu) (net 2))
 (segment (start 138.43 105.41) (end 138.43 107.315) (width 1.27) (layer F.Cu) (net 2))
 (segment (start 146.05 107.315) (end 146.05 105.41) (width 1.27) (layer F.Cu) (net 2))
 (segment (start 138.43 107.315) (end 146.05 107.315) (width 1.27) (layer F.Cu) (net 2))
 (segment (start 121.92 90.17) (end 124.46 90.17) (width 1.27) (layer B.Cu) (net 2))
 (segment (start 119.38 90.17) (end 121.92 90.17) (width 1.27) (layer B.Cu) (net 2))
 (segment (start 124.46 87.63) (end 124.46 90.17) (width 1.27) (layer B.Cu) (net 2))
 (segment (start 121.92 87.63) (end 121.92 90.17) (width 1.27) (layer B.Cu) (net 2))
 (segment (start 119.38 89.535) (end 119.38 90.17) (width 1.27) (layer B.Cu) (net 2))
 (segment (start 119.38 87.63) (end 119.38 89.535) (width 1.27) (layer B.Cu) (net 2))
 (segment (start 155.575 83.82) (end 160.02 83.82) (width 0.3048) (layer B.Cu) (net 2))
 (segment (start 160.02 83.82) (end 162.56 86.36) (width 0.3048) (layer B.Cu) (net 2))
 (segment (start 162.54 86.38) (end 162.54 91.44) (width 0.3048) (layer B.Cu) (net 2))
 (segment (start 162.56 86.36) (end 162.54 86.38) (width 0.3048) (layer B.Cu) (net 2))
 (segment (start 163.79 91.44) (end 162.54 91.44) (width 0.3048) (layer B.Cu) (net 2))
 (segment (start 155.575 83.82) (end 153.67 85.725) (width 0.3048) (layer B.Cu) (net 2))
 (segment (start 153.67 95.25) (end 151.13 97.79) (width 0.3048) (layer B.Cu) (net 2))
 (segment (start 153.67 85.725) (end 153.67 95.25) (width 0.3048) (layer B.Cu) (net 2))
 (segment (start 178.435 114.3) (end 175.895 114.3) (width 0.3048) (layer F.Cu) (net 3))
 (segment (start 175.895 114.3) (end 172.72 117.475) (width 0.3048) (layer F.Cu) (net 3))
 (segment (start 163.195 117.475) (end 162.56 118.11) (width 0.3048) (layer F.Cu) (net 3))
 (segment (start 172.72 117.475) (end 163.195 117.475) (width 0.3048) (layer F.Cu) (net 3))
 (segment (start 162.56 118.11) (end 162.56 119.38) (width 0.3048) (layer F.Cu) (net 3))
 (segment (start 153.67 115.57) (end 148.59 110.49) (width 0.3048) (layer B.Cu) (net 3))
 (segment (start 148.59 110.49) (end 148.59 105.41) (width 0.3048) (layer B.Cu) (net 3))
 (segment (start 159.863551 115.57) (end 153.67 115.57) (width 0.3048) (layer B.Cu) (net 3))
 (segment (start 162.56 119.38) (end 162.56 118.266449) (width 0.3048) (layer B.Cu) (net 3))
 (segment (start 162.56 118.266449) (end 159.863551 115.57) (width 0.3048) (layer B.Cu) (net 3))
 (segment (start 116.84 90.17) (end 116.84 87.63) (width 1.27) (layer F.Cu) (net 3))
 (segment (start 116.84 100.33) (end 116.84 90.17) (width 1.27) (layer F.Cu) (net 3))
 (segment (start 120.015 103.505) (end 116.84 100.33) (width 1.27) (layer F.Cu) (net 3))
 (segment (start 147.798551 103.505) (end 120.015 103.505) (width 1.27) (layer F.Cu) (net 3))
 (segment (start 148.59 105.41) (end 148.59 104.296449) (width 1.27) (layer F.Cu) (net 3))
 (segment (start 148.59 104.296449) (end 147.798551 103.505) (width 1.27) (layer F.Cu) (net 3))
 (segment (start 151.13 105.41) (end 148.59 105.41) (width 1.27) (layer F.Cu) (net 3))
 (segment (start 151.13 93.98) (end 149.86 95.25) (width 0.3048) (layer B.Cu) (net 3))
 (segment (start 149.86 95.25) (end 149.86 100.33) (width 0.3048) (layer B.Cu) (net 3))
 (segment (start 149.86 100.33) (end 148.59 101.6) (width 0.3048) (layer B.Cu) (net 3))
 (segment (start 148.59 101.6) (end 148.59 105.41) (width 0.3048) (layer B.Cu) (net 3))
 (segment (start 138.9888 127.7112) (end 127 127.7112) (width 0.3048) (layer B.Cu) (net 4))
 (segment (start 147.142201 119.557799) (end 138.9888 127.7112) (width 0.3048) (layer B.Cu) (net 4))
 (segment (start 147.142201 96.697799) (end 147.142201 119.557799) (width 0.3048) (layer B.Cu) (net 4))
 (segment (start 148.59 93.98) (end 148.59 95.25) (width 0.3048) (layer B.Cu) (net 4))
 (segment (start 148.59 95.25) (end 147.142201 96.697799) (width 0.3048) (layer B.Cu) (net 4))
 (segment (start 154.94 119.38) (end 152.4 121.92) (width 0.3048) (layer B.Cu) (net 5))
 (segment (start 152.4 121.92) (end 152.4 127.7112) (width 0.3048) (layer B.Cu) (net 5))
 (segment (start 140.97 121.285) (end 140.97 119.38) (width 0.3048) (layer F.Cu) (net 6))
 (segment (start 142.875 123.19) (end 140.97 121.285) (width 0.3048) (layer F.Cu) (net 6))
 (segment (start 158.115 123.19) (end 142.875 123.19) (width 0.3048) (layer F.Cu) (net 6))
 (segment (start 162.6362 127.7112) (end 158.115 123.19) (width 0.3048) (layer F.Cu) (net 6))
 (segment (start 177.8 127.7112) (end 162.6362 127.7112) (width 0.3048) (layer F.Cu) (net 6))
 (segment (start 155.72017 102.390638) (end 154.932771 101.603239) (width 0.3048) (layer F.Cu) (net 7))
 (segment (start 157.387352 102.390638) (end 155.72017 102.390638) (width 0.3048) (layer F.Cu) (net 7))
 (segment (start 166.344601 101.625399) (end 158.152591 101.625399) (width 0.3048) (layer F.Cu) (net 7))
 (segment (start 158.152591 101.625399) (end 157.387352 102.390638) (width 0.3048) (layer F.Cu) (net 7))
 (segment (start 170.18 97.79) (end 166.344601 101.625399) (width 0.3048) (layer F.Cu) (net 7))
 (segment (start 154.929532 101.6) (end 154.932771 101.603239) (width 0.3048) (layer F.Cu) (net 7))
 (segment (start 154.94 97.79) (end 154.94 101.59601) (width 0.3048) (layer B.Cu) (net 7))
 (segment (start 143.51 101.6) (end 154.929532 101.6) (width 0.3048) (layer F.Cu) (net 7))
 (segment (start 154.94 101.59601) (end 154.932771 101.603239) (width 0.3048) (layer B.Cu) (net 7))
 (via (at 154.932771 101.603239) (size 1.5748) (drill 0.9144) (layers F.Cu B.Cu) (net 7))
 (segment (start 143.51 105.41) (end 143.51 101.6) (width 0.3048) (layer B.Cu) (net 7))
 (via (at 143.51 101.6) (size 1.5748) (drill 0.9144) (layers F.Cu B.Cu) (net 7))
 (segment (start 143.51 105.41) (end 143.51 109.22) (width 0.3048) (layer B.Cu) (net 7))
 (segment (start 154.94 104.3178) (end 154.94 105.41) (width 0.3048) (layer B.Cu) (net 8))
 (segment (start 156.21 99.757988) (end 156.06855 99.899438) (width 0.3048) (layer B.Cu) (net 8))
 (segment (start 156.06855 101.094258) (end 156.21 101.235708) (width 0.3048) (layer B.Cu) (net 8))
 (segment (start 158.79 91.44) (end 158.79 93.94) (width 0.3048) (layer B.Cu) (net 8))
 (segment (start 156.21 101.235708) (end 156.21 103.0478) (width 0.3048) (layer B.Cu) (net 8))
 (segment (start 156.06855 99.899438) (end 156.06855 101.094258) (width 0.3048) (layer B.Cu) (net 8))
 (segment (start 158.79 93.94) (end 156.21 96.52) (width 0.3048) (layer B.Cu) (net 8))
 (segment (start 156.21 96.52) (end 156.21 99.757988) (width 0.3048) (layer B.Cu) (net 8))
 (segment (start 156.21 103.0478) (end 154.94 104.3178) (width 0.3048) (layer B.Cu) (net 8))
 (segment (start 156.21 104.14) (end 154.94 105.41) (width 0.3048) (layer F.Cu) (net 8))
 (segment (start 167.483551 104.14) (end 156.21 104.14) (width 0.3048) (layer F.Cu) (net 8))
 (segment (start 167.64 105.41) (end 167.64 104.296449) (width 0.3048) (layer F.Cu) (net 8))
 (segment (start 167.64 104.296449) (end 167.483551 104.14) (width 0.3048) (layer F.Cu) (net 8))
 (segment (start 154.94 109.22) (end 154.94 105.41) (width 0.3048) (layer B.Cu) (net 8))
 (segment (start 157.48 97.79) (end 157.48 95.885) (width 0.3048) (layer F.Cu) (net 9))
 (segment (start 157.48 95.885) (end 155.575 93.98) (width 0.3048) (layer F.Cu) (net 9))
 (segment (start 157.48 97.79) (end 157.48 98.903551) (width 0.3048) (layer B.Cu) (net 9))
 (segment (start 160.02 109.22) (end 157.48 109.22) (width 0.3048) (layer F.Cu) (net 10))
 (segment (start 164.933152 100.496848) (end 158.426703 100.496848) (width 0.3048) (layer F.Cu) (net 10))
 (segment (start 167.64 97.79) (end 164.933152 100.496848) (width 0.3048) (layer F.Cu) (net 10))
 (segment (start 157.48 100.663696) (end 157.313152 100.496848) (width 0.3048) (layer B.Cu) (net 10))
 (segment (start 158.426703 100.496848) (end 157.313152 100.496848) (width 0.3048) (layer F.Cu) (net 10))
 (segment (start 157.48 105.41) (end 157.48 100.663696) (width 0.3048) (layer B.Cu) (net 10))
 (via (at 157.313152 100.496848) (size 1.5748) (drill 0.9144) (layers F.Cu B.Cu) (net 10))
 (segment (start 157.48 109.22) (end 157.48 105.41) (width 0.3048) (layer B.Cu) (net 10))
 (segment (start 160.04 91.44) (end 160.04 97.77) (width 0.3048) (layer B.Cu) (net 11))
 (segment (start 160.04 97.77) (end 160.02 97.79) (width 0.3048) (layer B.Cu) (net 11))
 (segment (start 160.02 97.79) (end 160.02 105.41) (width 0.3048) (layer B.Cu) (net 11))
 (segment (start 162.56 109.22) (end 162.56 107.95) (width 0.3048) (layer B.Cu) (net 11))
 (segment (start 162.56 107.95) (end 160.02 105.41) (width 0.3048) (layer B.Cu) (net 11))
 (segment (start 168.91 93.98) (end 165.1 97.79) (width 0.3048) (layer B.Cu) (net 12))
 (segment (start 162.56 102.235) (end 162.56 105.41) (width 0.3048) (layer B.Cu) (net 12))
 (segment (start 165.1 99.695) (end 162.56 102.235) (width 0.3048) (layer B.Cu) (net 12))
 (segment (start 165.1 97.79) (end 165.1 99.695) (width 0.3048) (layer B.Cu) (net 12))
 (segment (start 166.37 93.98) (end 162.7632 93.98) (width 0.3048) (layer B.Cu) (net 14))
 (segment (start 162.7632 93.98) (end 161.29 92.5068) (width 0.3048) (layer B.Cu) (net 14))
 (segment (start 161.29 92.5068) (end 161.29 91.44) (width 0.3048) (layer B.Cu) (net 14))
 (segment (start 140.97 109.22) (end 140.97 113.03) (width 0.3048) (layer B.Cu) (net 16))
 (segment (start 143.51 115.57) (end 143.51 119.38) (width 0.3048) (layer B.Cu) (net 16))
 (segment (start 140.97 113.03) (end 143.51 115.57) (width 0.3048) (layer B.Cu) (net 16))
 (segment (start 140.97 105.41) (end 140.97 109.22) (width 0.3048) (layer B.Cu) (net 16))
 (segment (start 167.64 109.22) (end 165.1 109.22) (width 0.3048) (layer F.Cu) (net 13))
 (segment (start 165.1 105.41) (end 165.1 109.22) (width 0.3048) (layer B.Cu) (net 13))
 (segment (start 175.895 118.11) (end 175.895 116.84) (width 0.3048) (layer F.Cu) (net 19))
 (segment (start 174.625 119.38) (end 175.895 118.11) (width 0.3048) (layer F.Cu) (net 19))
 (segment (start 167.64 119.38) (end 174.625 119.38) (width 0.3048) (layer F.Cu) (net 19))
 (segment (start 151.13 83.82) (end 148.59 83.82) (width 0.3048) (layer F.Cu) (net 17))
 (segment (start 148.59 83.82) (end 146.05 83.82) (width 0.3048) (layer F.Cu) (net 17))
 (segment (start 140.97 83.82) (end 142.24 85.09) (width 0.3048) (layer F.Cu) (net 17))
 (segment (start 142.24 85.09) (end 144.78 85.09) (width 0.3048) (layer F.Cu) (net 17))
 (segment (start 144.78 85.09) (end 146.05 83.82) (width 0.3048) (layer F.Cu) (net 17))
 (segment (start 144.957799 84.912201) (end 144.957799 89.992201) (width 0.3048) (layer B.Cu) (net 17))
 (segment (start 146.05 83.82) (end 144.957799 84.912201) (width 0.3048) (layer B.Cu) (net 17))
 (segment (start 144.957799 89.992201) (end 147.32 92.354402) (width 0.3048) (layer B.Cu) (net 17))
 (segment (start 147.32 92.354402) (end 147.32 95.25) (width 0.3048) (layer B.Cu) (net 17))
 (segment (start 147.32 95.25) (end 146.05 96.52) (width 0.3048) (layer B.Cu) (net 17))
 (segment (start 146.05 96.52) (end 146.05 97.79) (width 0.3048) (layer B.Cu) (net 17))
 (segment (start 146.05 93.98) (end 143.51 93.98) (width 0.3048) (layer F.Cu) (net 15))
 (segment (start 146.05 93.98) (end 144.78 95.25) (width 0.3048) (layer B.Cu) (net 15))
 (segment (start 144.78 109.566458) (end 146.05 110.836458) (width 0.3048) (layer B.Cu) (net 15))
 (segment (start 144.78 95.25) (end 144.78 109.566458) (width 0.3048) (layer B.Cu) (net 15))
 (via (at 146.05 117.475) (size 1.5748) (drill 0.9144) (layers F.Cu B.Cu) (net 15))
 (segment (start 146.05 110.836458) (end 146.05 117.475) (width 0.3048) (layer B.Cu) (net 15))
 (segment (start 155.575 117.475) (end 157.48 119.38) (width 0.3048) (layer F.Cu) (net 15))
 (segment (start 146.05 117.475) (end 155.575 117.475) (width 0.3048) (layer F.Cu) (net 15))
 (segment (start 140.97 95.25) (end 143.186704 97.466704) (width 0.3048) (layer B.Cu) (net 18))
 (segment (start 140.97 93.98) (end 140.97 95.25) (width 0.3048) (layer B.Cu) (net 18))
 (segment (start 140.97 93.98) (end 140.97 90.17) (width 0.3048) (layer B.Cu) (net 18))
 (segment (start 140.97 90.17) (end 143.51 87.63) (width 0.3048) (layer B.Cu) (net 18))
 (segment (start 143.51 87.63) (end 143.51 83.82) (width 0.3048) (layer B.Cu) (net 18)))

